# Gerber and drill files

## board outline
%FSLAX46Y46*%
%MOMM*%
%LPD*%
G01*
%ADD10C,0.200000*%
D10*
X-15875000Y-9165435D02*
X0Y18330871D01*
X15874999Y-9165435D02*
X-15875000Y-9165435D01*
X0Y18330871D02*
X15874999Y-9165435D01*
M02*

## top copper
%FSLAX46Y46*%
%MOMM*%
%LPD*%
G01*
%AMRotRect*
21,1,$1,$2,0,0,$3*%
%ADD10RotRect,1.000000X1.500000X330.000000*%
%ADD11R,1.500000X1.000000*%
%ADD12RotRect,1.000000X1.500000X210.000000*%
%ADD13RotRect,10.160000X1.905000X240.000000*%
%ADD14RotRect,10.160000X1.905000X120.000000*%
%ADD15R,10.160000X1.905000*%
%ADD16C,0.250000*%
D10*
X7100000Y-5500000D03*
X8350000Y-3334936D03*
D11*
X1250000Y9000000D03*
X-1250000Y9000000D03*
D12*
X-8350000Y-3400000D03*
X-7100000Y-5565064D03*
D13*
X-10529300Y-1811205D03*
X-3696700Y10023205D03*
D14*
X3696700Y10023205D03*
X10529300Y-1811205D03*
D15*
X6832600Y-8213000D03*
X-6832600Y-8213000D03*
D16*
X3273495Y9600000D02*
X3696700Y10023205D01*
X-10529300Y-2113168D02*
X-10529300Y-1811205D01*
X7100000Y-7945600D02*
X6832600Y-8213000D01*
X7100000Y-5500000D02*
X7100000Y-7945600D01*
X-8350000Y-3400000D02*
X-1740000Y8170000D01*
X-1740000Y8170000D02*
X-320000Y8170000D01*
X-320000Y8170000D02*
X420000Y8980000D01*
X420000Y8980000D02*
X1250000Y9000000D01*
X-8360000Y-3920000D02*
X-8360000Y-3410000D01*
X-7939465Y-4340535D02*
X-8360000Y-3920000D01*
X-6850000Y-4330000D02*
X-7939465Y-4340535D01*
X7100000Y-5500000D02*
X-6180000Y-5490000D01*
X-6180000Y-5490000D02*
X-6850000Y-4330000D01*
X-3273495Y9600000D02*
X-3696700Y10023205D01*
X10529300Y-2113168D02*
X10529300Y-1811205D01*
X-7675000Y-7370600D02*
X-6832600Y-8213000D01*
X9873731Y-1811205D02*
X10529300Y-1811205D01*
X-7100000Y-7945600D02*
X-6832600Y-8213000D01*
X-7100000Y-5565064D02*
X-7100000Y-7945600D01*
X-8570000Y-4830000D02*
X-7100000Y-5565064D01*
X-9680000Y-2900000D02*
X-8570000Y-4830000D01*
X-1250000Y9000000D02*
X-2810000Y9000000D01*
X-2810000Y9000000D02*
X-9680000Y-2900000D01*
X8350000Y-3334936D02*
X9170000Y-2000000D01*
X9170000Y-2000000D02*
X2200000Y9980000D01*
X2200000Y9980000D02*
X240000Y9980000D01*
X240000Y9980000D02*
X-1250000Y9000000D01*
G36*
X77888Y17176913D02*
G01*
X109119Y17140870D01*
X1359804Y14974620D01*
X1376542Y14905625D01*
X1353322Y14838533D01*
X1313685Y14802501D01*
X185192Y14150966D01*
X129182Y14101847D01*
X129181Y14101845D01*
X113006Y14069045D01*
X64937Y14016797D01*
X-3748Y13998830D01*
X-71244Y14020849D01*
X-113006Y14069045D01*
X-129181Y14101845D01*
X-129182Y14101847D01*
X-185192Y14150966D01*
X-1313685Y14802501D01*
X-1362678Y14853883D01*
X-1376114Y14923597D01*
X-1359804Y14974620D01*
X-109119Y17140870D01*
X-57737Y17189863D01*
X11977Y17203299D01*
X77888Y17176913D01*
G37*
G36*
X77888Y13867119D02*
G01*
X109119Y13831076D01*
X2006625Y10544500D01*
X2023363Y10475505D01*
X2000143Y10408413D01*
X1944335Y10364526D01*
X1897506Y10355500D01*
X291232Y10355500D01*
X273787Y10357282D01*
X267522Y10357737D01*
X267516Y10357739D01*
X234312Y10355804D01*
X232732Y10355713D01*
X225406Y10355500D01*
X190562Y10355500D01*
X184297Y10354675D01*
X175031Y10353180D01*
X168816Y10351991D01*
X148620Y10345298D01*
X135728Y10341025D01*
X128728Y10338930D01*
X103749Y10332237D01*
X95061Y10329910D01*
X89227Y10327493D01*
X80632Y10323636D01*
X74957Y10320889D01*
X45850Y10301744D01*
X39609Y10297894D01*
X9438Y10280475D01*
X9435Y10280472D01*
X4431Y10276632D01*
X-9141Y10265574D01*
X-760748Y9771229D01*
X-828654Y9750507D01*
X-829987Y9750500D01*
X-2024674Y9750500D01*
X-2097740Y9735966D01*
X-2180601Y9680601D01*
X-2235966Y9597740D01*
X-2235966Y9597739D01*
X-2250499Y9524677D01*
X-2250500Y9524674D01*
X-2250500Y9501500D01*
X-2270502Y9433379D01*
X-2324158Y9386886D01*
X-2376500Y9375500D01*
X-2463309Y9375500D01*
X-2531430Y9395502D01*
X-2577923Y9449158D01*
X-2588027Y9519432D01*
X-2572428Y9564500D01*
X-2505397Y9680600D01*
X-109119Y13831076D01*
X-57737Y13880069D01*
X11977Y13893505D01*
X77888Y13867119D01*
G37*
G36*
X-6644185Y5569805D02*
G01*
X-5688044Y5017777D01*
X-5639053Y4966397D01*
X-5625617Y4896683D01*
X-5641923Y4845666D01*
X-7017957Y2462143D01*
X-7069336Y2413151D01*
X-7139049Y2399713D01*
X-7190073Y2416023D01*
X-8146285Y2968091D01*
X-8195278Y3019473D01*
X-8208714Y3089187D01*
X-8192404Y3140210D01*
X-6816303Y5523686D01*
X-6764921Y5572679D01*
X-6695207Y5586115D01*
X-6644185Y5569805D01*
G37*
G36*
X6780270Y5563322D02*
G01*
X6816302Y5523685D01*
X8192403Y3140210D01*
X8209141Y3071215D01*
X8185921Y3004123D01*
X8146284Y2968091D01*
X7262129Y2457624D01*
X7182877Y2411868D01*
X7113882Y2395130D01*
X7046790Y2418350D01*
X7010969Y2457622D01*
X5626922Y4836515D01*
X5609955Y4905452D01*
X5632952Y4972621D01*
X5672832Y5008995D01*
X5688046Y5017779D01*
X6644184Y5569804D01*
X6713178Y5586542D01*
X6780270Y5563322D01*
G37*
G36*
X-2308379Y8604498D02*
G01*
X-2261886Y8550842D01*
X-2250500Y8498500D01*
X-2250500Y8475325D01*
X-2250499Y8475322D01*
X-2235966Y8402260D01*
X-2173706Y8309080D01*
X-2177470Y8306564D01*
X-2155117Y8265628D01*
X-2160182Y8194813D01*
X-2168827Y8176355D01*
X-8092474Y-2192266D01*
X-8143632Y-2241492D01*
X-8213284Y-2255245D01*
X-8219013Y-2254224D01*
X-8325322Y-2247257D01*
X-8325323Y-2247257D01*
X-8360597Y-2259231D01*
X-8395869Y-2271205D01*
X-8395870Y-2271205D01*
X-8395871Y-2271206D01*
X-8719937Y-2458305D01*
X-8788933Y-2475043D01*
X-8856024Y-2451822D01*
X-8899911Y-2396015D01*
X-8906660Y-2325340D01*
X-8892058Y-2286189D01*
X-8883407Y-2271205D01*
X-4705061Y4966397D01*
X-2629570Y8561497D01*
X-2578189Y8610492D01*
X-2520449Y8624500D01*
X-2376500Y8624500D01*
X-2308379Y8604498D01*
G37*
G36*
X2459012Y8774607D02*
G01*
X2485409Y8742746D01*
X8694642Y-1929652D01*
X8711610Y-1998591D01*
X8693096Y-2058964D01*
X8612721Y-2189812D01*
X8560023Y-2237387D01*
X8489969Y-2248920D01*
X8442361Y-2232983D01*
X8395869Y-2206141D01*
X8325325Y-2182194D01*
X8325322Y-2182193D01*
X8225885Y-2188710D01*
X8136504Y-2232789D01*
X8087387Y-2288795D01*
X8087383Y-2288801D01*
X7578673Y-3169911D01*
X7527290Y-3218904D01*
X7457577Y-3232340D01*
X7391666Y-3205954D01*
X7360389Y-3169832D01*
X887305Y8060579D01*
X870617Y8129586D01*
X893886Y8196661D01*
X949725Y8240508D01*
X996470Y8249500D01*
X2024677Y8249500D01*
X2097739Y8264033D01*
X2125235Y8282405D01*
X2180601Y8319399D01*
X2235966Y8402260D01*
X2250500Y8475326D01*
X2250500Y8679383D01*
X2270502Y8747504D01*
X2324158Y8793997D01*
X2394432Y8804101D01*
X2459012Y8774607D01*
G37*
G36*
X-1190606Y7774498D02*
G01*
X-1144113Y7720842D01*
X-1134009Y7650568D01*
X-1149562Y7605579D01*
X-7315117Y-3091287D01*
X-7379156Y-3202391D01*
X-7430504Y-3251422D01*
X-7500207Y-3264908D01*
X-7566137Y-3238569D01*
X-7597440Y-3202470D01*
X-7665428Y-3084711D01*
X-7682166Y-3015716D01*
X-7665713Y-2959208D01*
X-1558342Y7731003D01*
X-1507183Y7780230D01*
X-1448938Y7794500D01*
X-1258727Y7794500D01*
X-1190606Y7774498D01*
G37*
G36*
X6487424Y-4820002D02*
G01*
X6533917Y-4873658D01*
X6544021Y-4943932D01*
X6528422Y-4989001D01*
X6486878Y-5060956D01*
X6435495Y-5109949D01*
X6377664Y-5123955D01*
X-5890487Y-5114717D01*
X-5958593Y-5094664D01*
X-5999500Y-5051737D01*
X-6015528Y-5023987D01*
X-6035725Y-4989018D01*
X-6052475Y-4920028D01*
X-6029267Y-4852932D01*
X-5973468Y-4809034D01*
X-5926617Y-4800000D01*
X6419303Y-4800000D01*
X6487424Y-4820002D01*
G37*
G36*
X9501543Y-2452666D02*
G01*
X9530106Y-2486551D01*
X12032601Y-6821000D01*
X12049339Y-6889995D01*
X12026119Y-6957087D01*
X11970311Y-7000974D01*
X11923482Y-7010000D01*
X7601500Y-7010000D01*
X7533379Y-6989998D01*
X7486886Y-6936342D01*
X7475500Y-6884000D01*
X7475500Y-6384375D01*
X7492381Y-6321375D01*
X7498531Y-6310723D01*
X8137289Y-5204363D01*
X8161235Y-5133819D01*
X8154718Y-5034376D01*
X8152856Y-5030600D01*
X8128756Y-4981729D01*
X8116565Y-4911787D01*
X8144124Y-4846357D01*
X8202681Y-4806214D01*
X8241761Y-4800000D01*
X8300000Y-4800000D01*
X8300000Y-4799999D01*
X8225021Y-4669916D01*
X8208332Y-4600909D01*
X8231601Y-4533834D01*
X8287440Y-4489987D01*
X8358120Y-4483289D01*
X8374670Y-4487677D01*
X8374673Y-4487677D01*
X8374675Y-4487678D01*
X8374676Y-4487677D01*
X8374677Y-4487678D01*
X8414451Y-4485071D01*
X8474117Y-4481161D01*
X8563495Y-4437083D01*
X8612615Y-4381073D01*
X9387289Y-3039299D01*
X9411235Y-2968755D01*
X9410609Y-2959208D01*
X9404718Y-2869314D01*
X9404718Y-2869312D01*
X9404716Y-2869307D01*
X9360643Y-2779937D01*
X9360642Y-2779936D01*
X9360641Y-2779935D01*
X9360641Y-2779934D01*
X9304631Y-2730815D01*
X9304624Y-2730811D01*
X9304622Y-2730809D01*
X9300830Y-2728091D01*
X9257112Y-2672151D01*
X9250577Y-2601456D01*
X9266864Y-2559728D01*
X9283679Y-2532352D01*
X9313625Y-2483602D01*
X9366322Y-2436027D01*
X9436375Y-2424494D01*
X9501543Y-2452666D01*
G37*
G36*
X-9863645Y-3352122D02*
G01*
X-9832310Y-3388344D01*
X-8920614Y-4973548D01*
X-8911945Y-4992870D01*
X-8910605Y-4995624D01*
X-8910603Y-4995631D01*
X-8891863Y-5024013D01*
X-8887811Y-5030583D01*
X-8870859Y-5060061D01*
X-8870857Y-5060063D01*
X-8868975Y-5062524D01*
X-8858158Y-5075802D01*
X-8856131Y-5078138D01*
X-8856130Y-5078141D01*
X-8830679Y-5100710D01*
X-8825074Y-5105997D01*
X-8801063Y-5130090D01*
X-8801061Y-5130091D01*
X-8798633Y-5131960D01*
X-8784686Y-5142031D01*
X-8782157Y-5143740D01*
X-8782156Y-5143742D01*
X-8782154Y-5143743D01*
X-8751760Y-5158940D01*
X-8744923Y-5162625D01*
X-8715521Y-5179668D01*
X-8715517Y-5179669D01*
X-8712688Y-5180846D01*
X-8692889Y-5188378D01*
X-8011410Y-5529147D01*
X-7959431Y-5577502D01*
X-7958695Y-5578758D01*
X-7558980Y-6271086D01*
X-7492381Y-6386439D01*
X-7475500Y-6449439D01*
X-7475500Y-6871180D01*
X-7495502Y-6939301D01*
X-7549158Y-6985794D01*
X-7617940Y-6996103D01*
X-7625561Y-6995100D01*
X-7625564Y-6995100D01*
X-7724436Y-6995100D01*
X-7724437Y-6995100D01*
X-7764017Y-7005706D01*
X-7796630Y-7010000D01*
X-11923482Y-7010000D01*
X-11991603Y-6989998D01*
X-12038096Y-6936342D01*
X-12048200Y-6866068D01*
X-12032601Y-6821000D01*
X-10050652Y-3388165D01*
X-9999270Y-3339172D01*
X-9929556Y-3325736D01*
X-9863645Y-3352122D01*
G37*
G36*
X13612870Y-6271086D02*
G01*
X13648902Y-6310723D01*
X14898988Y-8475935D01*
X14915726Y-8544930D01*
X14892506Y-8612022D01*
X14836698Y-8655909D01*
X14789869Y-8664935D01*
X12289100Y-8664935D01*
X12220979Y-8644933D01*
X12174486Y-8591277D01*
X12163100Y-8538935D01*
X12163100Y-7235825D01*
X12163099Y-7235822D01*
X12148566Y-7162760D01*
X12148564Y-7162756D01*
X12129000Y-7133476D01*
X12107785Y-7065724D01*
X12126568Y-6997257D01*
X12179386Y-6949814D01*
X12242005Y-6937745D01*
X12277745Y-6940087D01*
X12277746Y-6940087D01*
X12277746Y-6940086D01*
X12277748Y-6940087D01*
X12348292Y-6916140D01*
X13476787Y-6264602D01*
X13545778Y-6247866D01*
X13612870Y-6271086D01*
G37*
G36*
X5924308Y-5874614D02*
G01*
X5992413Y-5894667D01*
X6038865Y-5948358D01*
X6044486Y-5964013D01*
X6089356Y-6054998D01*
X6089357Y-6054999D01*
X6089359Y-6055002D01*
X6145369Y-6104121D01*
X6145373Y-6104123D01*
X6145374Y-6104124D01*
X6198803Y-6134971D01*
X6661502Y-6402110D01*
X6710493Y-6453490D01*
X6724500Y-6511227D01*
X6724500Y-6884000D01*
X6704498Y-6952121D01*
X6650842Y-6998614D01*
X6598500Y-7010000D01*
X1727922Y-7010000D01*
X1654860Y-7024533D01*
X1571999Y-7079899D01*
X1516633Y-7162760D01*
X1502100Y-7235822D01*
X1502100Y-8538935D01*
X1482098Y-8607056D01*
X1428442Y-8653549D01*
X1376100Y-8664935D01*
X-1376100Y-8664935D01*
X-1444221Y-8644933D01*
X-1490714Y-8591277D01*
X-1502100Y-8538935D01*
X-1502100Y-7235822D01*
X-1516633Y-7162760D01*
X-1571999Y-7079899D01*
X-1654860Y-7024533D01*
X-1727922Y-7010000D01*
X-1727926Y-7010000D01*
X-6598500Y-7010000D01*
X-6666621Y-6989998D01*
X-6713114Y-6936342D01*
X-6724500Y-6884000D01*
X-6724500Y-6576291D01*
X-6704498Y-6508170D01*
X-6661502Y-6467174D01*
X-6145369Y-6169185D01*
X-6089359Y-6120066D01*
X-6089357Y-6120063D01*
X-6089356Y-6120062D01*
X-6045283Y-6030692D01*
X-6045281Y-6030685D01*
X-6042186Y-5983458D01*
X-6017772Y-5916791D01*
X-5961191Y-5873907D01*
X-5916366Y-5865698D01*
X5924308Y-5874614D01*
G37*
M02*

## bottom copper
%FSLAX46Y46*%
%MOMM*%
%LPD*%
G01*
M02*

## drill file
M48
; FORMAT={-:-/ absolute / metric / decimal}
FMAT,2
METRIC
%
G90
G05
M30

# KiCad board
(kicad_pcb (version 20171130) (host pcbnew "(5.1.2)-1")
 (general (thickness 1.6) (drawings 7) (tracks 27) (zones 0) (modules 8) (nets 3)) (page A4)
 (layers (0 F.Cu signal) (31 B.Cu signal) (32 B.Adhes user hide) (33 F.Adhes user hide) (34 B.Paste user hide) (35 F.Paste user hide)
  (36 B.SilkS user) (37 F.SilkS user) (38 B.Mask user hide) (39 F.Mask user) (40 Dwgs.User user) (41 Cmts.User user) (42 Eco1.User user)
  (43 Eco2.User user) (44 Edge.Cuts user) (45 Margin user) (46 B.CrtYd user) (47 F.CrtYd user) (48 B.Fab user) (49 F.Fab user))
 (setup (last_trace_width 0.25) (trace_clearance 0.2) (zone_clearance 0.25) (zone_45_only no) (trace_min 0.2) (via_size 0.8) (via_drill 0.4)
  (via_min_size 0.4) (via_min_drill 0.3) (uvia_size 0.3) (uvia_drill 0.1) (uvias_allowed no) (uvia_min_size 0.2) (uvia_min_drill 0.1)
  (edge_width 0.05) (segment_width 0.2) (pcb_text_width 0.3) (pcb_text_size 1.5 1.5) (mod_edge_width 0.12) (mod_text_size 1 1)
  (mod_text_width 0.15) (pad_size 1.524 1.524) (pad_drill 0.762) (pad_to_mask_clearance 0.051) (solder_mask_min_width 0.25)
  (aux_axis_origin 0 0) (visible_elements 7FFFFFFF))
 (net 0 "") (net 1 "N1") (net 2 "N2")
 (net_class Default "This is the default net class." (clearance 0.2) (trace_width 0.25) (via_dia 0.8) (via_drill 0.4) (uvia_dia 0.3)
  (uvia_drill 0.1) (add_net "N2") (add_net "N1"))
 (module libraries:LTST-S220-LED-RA (layer F.Cu) (at 7.725 4.417468 330)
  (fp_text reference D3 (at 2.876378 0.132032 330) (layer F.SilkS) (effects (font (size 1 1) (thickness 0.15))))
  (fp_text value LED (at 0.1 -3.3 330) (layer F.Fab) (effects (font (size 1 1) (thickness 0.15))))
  (pad 1 smd rect (at 0 1.25 330) (size 1 1.5) (layers F.Cu F.Paste F.Mask) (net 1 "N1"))
  (pad 2 smd rect (at 0 -1.25 330) (size 1 1.5) (layers F.Cu F.Paste F.Mask) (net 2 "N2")))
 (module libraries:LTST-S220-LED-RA (layer F.Cu) (at 0 -9 90)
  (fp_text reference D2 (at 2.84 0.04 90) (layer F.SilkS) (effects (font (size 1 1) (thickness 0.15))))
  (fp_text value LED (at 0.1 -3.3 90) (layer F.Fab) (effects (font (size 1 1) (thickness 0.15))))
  (pad 1 smd rect (at 0 1.25 90) (size 1 1.5) (layers F.Cu F.Paste F.Mask) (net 1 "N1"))
  (pad 2 smd rect (at 0 -1.25 90) (size 1 1.5) (layers F.Cu F.Paste F.Mask) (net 2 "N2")))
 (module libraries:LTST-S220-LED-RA (layer F.Cu) (at -7.725 4.482532 210)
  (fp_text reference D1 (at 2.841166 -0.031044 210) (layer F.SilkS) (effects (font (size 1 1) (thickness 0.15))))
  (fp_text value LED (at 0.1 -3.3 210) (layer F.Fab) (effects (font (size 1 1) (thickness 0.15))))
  (pad 1 smd rect (at 0 1.25 210) (size 1 1.5) (layers F.Cu F.Paste F.Mask) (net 1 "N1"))
  (pad 2 smd rect (at 0 -1.25 210) (size 1 1.5) (layers F.Cu F.Paste F.Mask) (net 2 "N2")))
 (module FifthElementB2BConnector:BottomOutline (layer F.Cu) (at 0 0)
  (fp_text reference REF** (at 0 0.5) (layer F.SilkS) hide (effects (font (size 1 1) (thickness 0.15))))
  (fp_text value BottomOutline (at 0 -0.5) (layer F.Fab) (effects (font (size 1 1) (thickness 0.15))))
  (fp_line (start -15.875 9.165435) (end 0 -18.330871) (layer Edge.Cuts) (width 0.2))
  (fp_line (start 15.874999 9.165435) (end -15.875 9.165435) (layer Edge.Cuts) (width 0.2))
  (fp_line (start 0 -18.330871) (end 15.874999 9.165435) (layer Edge.Cuts) (width 0.2)))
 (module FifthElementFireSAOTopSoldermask (layer B.Cu) (at 0 -4.6 180)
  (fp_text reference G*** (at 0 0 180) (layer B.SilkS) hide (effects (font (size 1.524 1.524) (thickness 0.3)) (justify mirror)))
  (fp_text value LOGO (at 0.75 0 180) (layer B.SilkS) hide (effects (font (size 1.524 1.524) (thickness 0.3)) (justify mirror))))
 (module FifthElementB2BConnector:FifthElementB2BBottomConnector (layer F.Cu) (at -7.113 -4.106 240)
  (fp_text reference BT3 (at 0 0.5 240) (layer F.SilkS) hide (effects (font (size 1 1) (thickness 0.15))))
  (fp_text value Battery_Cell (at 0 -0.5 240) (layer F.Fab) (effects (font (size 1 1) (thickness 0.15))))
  (pad 2 smd rect (at 6.8326 0 240) (size 10.16 1.905) (layers F.Cu F.Paste F.Mask) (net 1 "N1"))
  (pad 1 smd rect (at -6.8326 0 240) (size 10.16 1.905) (layers F.Cu F.Paste F.Mask) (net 2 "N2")))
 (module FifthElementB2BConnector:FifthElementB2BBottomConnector (layer F.Cu) (at 7.113 -4.106 120)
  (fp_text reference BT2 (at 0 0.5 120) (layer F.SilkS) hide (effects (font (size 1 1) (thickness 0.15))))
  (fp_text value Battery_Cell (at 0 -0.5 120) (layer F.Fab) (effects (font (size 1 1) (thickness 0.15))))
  (pad 2 smd rect (at 6.8326 0 120) (size 10.16 1.905) (layers F.Cu F.Paste F.Mask) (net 1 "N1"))
  (pad 1 smd rect (at -6.8326 0 120) (size 10.16 1.905) (layers F.Cu F.Paste F.Mask) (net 2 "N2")))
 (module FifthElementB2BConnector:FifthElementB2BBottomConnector (layer F.Cu) (at 0 8.213)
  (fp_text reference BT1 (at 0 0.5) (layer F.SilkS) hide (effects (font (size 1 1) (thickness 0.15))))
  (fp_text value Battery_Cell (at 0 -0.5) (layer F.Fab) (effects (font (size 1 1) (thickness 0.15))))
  (pad 2 smd rect (at 6.8326 0) (size 10.16 1.905) (layers F.Cu F.Paste F.Mask) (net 1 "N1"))
  (pad 1 smd rect (at -6.8326 0) (size 10.16 1.905) (layers F.Cu F.Paste F.Mask) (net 2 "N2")))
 (segment (start 3.273495 -9.6) (end 3.6967 -10.023205) (width 0.25) (layer F.Cu) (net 1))
 (segment (start -10.5293 2.113168) (end -10.5293 1.811205) (width 0.25) (layer F.Cu) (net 1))
 (segment (start 7.1 7.9456) (end 6.8326 8.213) (width 0.25) (layer F.Cu) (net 1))
 (segment (start 7.1 5.5) (end 7.1 7.9456) (width 0.25) (layer F.Cu) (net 1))
 (segment (start -8.35 3.4) (end -1.74 -8.17) (width 0.25) (layer F.Cu) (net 1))
 (segment (start -1.74 -8.17) (end -0.32 -8.17) (width 0.25) (layer F.Cu) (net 1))
 (segment (start -0.32 -8.17) (end 0.42 -8.98) (width 0.25) (layer F.Cu) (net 1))
 (segment (start 0.42 -8.98) (end 1.25 -9) (width 0.25) (layer F.Cu) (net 1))
 (segment (start -8.36 3.92) (end -8.36 3.41) (width 0.25) (layer F.Cu) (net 1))
 (segment (start -7.939465 4.340535) (end -8.36 3.92) (width 0.25) (layer F.Cu) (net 1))
 (segment (start -6.85 4.33) (end -7.939465 4.340535) (width 0.25) (layer F.Cu) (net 1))
 (segment (start 7.1 5.5) (end -6.18 5.49) (width 0.25) (layer F.Cu) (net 1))
 (segment (start -6.18 5.49) (end -6.85 4.33) (width 0.25) (layer F.Cu) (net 1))
 (segment (start -3.273495 -9.6) (end -3.6967 -10.023205) (width 0.25) (layer F.Cu) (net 2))
 (segment (start 10.5293 2.113168) (end 10.5293 1.811205) (width 0.25) (layer F.Cu) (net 2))
 (segment (start -7.675 7.3706) (end -6.8326 8.213) (width 0.25) (layer F.Cu) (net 2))
 (segment (start 9.873731 1.811205) (end 10.5293 1.811205) (width 0.25) (layer F.Cu) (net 2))
 (segment (start -7.1 7.9456) (end -6.8326 8.213) (width 0.25) (layer F.Cu) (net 2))
 (segment (start -7.1 5.565064) (end -7.1 7.9456) (width 0.25) (layer F.Cu) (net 2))
 (segment (start -8.57 4.83) (end -7.1 5.565064) (width 0.25) (layer F.Cu) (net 2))
 (segment (start -9.68 2.9) (end -8.57 4.83) (width 0.25) (layer F.Cu) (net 2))
 (segment (start -1.25 -9) (end -2.81 -9) (width 0.25) (layer F.Cu) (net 2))
 (segment (start -2.81 -9) (end -9.68 2.9) (width 0.25) (layer F.Cu) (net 2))
 (segment (start 8.35 3.334936) (end 9.17 2) (width 0.25) (layer F.Cu) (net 2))
 (segment (start 9.17 2) (end 2.2 -9.98) (width 0.25) (layer F.Cu) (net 2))
 (segment (start 2.2 -9.98) (end 0.24 -9.98) (width 0.25) (layer F.Cu) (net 2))
 (segment (start 0.24 -9.98) (end -1.25 -9) (width 0.25) (layer F.Cu) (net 2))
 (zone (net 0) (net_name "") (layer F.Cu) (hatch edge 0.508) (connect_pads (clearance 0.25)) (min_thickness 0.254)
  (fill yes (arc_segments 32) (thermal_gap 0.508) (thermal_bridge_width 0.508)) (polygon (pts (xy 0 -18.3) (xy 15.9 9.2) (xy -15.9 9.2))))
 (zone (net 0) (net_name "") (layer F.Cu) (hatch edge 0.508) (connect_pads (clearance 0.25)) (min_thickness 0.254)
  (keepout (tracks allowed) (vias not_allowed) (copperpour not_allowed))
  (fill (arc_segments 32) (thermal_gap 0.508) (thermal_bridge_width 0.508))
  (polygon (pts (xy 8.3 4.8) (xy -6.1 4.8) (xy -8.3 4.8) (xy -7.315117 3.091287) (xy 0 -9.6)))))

